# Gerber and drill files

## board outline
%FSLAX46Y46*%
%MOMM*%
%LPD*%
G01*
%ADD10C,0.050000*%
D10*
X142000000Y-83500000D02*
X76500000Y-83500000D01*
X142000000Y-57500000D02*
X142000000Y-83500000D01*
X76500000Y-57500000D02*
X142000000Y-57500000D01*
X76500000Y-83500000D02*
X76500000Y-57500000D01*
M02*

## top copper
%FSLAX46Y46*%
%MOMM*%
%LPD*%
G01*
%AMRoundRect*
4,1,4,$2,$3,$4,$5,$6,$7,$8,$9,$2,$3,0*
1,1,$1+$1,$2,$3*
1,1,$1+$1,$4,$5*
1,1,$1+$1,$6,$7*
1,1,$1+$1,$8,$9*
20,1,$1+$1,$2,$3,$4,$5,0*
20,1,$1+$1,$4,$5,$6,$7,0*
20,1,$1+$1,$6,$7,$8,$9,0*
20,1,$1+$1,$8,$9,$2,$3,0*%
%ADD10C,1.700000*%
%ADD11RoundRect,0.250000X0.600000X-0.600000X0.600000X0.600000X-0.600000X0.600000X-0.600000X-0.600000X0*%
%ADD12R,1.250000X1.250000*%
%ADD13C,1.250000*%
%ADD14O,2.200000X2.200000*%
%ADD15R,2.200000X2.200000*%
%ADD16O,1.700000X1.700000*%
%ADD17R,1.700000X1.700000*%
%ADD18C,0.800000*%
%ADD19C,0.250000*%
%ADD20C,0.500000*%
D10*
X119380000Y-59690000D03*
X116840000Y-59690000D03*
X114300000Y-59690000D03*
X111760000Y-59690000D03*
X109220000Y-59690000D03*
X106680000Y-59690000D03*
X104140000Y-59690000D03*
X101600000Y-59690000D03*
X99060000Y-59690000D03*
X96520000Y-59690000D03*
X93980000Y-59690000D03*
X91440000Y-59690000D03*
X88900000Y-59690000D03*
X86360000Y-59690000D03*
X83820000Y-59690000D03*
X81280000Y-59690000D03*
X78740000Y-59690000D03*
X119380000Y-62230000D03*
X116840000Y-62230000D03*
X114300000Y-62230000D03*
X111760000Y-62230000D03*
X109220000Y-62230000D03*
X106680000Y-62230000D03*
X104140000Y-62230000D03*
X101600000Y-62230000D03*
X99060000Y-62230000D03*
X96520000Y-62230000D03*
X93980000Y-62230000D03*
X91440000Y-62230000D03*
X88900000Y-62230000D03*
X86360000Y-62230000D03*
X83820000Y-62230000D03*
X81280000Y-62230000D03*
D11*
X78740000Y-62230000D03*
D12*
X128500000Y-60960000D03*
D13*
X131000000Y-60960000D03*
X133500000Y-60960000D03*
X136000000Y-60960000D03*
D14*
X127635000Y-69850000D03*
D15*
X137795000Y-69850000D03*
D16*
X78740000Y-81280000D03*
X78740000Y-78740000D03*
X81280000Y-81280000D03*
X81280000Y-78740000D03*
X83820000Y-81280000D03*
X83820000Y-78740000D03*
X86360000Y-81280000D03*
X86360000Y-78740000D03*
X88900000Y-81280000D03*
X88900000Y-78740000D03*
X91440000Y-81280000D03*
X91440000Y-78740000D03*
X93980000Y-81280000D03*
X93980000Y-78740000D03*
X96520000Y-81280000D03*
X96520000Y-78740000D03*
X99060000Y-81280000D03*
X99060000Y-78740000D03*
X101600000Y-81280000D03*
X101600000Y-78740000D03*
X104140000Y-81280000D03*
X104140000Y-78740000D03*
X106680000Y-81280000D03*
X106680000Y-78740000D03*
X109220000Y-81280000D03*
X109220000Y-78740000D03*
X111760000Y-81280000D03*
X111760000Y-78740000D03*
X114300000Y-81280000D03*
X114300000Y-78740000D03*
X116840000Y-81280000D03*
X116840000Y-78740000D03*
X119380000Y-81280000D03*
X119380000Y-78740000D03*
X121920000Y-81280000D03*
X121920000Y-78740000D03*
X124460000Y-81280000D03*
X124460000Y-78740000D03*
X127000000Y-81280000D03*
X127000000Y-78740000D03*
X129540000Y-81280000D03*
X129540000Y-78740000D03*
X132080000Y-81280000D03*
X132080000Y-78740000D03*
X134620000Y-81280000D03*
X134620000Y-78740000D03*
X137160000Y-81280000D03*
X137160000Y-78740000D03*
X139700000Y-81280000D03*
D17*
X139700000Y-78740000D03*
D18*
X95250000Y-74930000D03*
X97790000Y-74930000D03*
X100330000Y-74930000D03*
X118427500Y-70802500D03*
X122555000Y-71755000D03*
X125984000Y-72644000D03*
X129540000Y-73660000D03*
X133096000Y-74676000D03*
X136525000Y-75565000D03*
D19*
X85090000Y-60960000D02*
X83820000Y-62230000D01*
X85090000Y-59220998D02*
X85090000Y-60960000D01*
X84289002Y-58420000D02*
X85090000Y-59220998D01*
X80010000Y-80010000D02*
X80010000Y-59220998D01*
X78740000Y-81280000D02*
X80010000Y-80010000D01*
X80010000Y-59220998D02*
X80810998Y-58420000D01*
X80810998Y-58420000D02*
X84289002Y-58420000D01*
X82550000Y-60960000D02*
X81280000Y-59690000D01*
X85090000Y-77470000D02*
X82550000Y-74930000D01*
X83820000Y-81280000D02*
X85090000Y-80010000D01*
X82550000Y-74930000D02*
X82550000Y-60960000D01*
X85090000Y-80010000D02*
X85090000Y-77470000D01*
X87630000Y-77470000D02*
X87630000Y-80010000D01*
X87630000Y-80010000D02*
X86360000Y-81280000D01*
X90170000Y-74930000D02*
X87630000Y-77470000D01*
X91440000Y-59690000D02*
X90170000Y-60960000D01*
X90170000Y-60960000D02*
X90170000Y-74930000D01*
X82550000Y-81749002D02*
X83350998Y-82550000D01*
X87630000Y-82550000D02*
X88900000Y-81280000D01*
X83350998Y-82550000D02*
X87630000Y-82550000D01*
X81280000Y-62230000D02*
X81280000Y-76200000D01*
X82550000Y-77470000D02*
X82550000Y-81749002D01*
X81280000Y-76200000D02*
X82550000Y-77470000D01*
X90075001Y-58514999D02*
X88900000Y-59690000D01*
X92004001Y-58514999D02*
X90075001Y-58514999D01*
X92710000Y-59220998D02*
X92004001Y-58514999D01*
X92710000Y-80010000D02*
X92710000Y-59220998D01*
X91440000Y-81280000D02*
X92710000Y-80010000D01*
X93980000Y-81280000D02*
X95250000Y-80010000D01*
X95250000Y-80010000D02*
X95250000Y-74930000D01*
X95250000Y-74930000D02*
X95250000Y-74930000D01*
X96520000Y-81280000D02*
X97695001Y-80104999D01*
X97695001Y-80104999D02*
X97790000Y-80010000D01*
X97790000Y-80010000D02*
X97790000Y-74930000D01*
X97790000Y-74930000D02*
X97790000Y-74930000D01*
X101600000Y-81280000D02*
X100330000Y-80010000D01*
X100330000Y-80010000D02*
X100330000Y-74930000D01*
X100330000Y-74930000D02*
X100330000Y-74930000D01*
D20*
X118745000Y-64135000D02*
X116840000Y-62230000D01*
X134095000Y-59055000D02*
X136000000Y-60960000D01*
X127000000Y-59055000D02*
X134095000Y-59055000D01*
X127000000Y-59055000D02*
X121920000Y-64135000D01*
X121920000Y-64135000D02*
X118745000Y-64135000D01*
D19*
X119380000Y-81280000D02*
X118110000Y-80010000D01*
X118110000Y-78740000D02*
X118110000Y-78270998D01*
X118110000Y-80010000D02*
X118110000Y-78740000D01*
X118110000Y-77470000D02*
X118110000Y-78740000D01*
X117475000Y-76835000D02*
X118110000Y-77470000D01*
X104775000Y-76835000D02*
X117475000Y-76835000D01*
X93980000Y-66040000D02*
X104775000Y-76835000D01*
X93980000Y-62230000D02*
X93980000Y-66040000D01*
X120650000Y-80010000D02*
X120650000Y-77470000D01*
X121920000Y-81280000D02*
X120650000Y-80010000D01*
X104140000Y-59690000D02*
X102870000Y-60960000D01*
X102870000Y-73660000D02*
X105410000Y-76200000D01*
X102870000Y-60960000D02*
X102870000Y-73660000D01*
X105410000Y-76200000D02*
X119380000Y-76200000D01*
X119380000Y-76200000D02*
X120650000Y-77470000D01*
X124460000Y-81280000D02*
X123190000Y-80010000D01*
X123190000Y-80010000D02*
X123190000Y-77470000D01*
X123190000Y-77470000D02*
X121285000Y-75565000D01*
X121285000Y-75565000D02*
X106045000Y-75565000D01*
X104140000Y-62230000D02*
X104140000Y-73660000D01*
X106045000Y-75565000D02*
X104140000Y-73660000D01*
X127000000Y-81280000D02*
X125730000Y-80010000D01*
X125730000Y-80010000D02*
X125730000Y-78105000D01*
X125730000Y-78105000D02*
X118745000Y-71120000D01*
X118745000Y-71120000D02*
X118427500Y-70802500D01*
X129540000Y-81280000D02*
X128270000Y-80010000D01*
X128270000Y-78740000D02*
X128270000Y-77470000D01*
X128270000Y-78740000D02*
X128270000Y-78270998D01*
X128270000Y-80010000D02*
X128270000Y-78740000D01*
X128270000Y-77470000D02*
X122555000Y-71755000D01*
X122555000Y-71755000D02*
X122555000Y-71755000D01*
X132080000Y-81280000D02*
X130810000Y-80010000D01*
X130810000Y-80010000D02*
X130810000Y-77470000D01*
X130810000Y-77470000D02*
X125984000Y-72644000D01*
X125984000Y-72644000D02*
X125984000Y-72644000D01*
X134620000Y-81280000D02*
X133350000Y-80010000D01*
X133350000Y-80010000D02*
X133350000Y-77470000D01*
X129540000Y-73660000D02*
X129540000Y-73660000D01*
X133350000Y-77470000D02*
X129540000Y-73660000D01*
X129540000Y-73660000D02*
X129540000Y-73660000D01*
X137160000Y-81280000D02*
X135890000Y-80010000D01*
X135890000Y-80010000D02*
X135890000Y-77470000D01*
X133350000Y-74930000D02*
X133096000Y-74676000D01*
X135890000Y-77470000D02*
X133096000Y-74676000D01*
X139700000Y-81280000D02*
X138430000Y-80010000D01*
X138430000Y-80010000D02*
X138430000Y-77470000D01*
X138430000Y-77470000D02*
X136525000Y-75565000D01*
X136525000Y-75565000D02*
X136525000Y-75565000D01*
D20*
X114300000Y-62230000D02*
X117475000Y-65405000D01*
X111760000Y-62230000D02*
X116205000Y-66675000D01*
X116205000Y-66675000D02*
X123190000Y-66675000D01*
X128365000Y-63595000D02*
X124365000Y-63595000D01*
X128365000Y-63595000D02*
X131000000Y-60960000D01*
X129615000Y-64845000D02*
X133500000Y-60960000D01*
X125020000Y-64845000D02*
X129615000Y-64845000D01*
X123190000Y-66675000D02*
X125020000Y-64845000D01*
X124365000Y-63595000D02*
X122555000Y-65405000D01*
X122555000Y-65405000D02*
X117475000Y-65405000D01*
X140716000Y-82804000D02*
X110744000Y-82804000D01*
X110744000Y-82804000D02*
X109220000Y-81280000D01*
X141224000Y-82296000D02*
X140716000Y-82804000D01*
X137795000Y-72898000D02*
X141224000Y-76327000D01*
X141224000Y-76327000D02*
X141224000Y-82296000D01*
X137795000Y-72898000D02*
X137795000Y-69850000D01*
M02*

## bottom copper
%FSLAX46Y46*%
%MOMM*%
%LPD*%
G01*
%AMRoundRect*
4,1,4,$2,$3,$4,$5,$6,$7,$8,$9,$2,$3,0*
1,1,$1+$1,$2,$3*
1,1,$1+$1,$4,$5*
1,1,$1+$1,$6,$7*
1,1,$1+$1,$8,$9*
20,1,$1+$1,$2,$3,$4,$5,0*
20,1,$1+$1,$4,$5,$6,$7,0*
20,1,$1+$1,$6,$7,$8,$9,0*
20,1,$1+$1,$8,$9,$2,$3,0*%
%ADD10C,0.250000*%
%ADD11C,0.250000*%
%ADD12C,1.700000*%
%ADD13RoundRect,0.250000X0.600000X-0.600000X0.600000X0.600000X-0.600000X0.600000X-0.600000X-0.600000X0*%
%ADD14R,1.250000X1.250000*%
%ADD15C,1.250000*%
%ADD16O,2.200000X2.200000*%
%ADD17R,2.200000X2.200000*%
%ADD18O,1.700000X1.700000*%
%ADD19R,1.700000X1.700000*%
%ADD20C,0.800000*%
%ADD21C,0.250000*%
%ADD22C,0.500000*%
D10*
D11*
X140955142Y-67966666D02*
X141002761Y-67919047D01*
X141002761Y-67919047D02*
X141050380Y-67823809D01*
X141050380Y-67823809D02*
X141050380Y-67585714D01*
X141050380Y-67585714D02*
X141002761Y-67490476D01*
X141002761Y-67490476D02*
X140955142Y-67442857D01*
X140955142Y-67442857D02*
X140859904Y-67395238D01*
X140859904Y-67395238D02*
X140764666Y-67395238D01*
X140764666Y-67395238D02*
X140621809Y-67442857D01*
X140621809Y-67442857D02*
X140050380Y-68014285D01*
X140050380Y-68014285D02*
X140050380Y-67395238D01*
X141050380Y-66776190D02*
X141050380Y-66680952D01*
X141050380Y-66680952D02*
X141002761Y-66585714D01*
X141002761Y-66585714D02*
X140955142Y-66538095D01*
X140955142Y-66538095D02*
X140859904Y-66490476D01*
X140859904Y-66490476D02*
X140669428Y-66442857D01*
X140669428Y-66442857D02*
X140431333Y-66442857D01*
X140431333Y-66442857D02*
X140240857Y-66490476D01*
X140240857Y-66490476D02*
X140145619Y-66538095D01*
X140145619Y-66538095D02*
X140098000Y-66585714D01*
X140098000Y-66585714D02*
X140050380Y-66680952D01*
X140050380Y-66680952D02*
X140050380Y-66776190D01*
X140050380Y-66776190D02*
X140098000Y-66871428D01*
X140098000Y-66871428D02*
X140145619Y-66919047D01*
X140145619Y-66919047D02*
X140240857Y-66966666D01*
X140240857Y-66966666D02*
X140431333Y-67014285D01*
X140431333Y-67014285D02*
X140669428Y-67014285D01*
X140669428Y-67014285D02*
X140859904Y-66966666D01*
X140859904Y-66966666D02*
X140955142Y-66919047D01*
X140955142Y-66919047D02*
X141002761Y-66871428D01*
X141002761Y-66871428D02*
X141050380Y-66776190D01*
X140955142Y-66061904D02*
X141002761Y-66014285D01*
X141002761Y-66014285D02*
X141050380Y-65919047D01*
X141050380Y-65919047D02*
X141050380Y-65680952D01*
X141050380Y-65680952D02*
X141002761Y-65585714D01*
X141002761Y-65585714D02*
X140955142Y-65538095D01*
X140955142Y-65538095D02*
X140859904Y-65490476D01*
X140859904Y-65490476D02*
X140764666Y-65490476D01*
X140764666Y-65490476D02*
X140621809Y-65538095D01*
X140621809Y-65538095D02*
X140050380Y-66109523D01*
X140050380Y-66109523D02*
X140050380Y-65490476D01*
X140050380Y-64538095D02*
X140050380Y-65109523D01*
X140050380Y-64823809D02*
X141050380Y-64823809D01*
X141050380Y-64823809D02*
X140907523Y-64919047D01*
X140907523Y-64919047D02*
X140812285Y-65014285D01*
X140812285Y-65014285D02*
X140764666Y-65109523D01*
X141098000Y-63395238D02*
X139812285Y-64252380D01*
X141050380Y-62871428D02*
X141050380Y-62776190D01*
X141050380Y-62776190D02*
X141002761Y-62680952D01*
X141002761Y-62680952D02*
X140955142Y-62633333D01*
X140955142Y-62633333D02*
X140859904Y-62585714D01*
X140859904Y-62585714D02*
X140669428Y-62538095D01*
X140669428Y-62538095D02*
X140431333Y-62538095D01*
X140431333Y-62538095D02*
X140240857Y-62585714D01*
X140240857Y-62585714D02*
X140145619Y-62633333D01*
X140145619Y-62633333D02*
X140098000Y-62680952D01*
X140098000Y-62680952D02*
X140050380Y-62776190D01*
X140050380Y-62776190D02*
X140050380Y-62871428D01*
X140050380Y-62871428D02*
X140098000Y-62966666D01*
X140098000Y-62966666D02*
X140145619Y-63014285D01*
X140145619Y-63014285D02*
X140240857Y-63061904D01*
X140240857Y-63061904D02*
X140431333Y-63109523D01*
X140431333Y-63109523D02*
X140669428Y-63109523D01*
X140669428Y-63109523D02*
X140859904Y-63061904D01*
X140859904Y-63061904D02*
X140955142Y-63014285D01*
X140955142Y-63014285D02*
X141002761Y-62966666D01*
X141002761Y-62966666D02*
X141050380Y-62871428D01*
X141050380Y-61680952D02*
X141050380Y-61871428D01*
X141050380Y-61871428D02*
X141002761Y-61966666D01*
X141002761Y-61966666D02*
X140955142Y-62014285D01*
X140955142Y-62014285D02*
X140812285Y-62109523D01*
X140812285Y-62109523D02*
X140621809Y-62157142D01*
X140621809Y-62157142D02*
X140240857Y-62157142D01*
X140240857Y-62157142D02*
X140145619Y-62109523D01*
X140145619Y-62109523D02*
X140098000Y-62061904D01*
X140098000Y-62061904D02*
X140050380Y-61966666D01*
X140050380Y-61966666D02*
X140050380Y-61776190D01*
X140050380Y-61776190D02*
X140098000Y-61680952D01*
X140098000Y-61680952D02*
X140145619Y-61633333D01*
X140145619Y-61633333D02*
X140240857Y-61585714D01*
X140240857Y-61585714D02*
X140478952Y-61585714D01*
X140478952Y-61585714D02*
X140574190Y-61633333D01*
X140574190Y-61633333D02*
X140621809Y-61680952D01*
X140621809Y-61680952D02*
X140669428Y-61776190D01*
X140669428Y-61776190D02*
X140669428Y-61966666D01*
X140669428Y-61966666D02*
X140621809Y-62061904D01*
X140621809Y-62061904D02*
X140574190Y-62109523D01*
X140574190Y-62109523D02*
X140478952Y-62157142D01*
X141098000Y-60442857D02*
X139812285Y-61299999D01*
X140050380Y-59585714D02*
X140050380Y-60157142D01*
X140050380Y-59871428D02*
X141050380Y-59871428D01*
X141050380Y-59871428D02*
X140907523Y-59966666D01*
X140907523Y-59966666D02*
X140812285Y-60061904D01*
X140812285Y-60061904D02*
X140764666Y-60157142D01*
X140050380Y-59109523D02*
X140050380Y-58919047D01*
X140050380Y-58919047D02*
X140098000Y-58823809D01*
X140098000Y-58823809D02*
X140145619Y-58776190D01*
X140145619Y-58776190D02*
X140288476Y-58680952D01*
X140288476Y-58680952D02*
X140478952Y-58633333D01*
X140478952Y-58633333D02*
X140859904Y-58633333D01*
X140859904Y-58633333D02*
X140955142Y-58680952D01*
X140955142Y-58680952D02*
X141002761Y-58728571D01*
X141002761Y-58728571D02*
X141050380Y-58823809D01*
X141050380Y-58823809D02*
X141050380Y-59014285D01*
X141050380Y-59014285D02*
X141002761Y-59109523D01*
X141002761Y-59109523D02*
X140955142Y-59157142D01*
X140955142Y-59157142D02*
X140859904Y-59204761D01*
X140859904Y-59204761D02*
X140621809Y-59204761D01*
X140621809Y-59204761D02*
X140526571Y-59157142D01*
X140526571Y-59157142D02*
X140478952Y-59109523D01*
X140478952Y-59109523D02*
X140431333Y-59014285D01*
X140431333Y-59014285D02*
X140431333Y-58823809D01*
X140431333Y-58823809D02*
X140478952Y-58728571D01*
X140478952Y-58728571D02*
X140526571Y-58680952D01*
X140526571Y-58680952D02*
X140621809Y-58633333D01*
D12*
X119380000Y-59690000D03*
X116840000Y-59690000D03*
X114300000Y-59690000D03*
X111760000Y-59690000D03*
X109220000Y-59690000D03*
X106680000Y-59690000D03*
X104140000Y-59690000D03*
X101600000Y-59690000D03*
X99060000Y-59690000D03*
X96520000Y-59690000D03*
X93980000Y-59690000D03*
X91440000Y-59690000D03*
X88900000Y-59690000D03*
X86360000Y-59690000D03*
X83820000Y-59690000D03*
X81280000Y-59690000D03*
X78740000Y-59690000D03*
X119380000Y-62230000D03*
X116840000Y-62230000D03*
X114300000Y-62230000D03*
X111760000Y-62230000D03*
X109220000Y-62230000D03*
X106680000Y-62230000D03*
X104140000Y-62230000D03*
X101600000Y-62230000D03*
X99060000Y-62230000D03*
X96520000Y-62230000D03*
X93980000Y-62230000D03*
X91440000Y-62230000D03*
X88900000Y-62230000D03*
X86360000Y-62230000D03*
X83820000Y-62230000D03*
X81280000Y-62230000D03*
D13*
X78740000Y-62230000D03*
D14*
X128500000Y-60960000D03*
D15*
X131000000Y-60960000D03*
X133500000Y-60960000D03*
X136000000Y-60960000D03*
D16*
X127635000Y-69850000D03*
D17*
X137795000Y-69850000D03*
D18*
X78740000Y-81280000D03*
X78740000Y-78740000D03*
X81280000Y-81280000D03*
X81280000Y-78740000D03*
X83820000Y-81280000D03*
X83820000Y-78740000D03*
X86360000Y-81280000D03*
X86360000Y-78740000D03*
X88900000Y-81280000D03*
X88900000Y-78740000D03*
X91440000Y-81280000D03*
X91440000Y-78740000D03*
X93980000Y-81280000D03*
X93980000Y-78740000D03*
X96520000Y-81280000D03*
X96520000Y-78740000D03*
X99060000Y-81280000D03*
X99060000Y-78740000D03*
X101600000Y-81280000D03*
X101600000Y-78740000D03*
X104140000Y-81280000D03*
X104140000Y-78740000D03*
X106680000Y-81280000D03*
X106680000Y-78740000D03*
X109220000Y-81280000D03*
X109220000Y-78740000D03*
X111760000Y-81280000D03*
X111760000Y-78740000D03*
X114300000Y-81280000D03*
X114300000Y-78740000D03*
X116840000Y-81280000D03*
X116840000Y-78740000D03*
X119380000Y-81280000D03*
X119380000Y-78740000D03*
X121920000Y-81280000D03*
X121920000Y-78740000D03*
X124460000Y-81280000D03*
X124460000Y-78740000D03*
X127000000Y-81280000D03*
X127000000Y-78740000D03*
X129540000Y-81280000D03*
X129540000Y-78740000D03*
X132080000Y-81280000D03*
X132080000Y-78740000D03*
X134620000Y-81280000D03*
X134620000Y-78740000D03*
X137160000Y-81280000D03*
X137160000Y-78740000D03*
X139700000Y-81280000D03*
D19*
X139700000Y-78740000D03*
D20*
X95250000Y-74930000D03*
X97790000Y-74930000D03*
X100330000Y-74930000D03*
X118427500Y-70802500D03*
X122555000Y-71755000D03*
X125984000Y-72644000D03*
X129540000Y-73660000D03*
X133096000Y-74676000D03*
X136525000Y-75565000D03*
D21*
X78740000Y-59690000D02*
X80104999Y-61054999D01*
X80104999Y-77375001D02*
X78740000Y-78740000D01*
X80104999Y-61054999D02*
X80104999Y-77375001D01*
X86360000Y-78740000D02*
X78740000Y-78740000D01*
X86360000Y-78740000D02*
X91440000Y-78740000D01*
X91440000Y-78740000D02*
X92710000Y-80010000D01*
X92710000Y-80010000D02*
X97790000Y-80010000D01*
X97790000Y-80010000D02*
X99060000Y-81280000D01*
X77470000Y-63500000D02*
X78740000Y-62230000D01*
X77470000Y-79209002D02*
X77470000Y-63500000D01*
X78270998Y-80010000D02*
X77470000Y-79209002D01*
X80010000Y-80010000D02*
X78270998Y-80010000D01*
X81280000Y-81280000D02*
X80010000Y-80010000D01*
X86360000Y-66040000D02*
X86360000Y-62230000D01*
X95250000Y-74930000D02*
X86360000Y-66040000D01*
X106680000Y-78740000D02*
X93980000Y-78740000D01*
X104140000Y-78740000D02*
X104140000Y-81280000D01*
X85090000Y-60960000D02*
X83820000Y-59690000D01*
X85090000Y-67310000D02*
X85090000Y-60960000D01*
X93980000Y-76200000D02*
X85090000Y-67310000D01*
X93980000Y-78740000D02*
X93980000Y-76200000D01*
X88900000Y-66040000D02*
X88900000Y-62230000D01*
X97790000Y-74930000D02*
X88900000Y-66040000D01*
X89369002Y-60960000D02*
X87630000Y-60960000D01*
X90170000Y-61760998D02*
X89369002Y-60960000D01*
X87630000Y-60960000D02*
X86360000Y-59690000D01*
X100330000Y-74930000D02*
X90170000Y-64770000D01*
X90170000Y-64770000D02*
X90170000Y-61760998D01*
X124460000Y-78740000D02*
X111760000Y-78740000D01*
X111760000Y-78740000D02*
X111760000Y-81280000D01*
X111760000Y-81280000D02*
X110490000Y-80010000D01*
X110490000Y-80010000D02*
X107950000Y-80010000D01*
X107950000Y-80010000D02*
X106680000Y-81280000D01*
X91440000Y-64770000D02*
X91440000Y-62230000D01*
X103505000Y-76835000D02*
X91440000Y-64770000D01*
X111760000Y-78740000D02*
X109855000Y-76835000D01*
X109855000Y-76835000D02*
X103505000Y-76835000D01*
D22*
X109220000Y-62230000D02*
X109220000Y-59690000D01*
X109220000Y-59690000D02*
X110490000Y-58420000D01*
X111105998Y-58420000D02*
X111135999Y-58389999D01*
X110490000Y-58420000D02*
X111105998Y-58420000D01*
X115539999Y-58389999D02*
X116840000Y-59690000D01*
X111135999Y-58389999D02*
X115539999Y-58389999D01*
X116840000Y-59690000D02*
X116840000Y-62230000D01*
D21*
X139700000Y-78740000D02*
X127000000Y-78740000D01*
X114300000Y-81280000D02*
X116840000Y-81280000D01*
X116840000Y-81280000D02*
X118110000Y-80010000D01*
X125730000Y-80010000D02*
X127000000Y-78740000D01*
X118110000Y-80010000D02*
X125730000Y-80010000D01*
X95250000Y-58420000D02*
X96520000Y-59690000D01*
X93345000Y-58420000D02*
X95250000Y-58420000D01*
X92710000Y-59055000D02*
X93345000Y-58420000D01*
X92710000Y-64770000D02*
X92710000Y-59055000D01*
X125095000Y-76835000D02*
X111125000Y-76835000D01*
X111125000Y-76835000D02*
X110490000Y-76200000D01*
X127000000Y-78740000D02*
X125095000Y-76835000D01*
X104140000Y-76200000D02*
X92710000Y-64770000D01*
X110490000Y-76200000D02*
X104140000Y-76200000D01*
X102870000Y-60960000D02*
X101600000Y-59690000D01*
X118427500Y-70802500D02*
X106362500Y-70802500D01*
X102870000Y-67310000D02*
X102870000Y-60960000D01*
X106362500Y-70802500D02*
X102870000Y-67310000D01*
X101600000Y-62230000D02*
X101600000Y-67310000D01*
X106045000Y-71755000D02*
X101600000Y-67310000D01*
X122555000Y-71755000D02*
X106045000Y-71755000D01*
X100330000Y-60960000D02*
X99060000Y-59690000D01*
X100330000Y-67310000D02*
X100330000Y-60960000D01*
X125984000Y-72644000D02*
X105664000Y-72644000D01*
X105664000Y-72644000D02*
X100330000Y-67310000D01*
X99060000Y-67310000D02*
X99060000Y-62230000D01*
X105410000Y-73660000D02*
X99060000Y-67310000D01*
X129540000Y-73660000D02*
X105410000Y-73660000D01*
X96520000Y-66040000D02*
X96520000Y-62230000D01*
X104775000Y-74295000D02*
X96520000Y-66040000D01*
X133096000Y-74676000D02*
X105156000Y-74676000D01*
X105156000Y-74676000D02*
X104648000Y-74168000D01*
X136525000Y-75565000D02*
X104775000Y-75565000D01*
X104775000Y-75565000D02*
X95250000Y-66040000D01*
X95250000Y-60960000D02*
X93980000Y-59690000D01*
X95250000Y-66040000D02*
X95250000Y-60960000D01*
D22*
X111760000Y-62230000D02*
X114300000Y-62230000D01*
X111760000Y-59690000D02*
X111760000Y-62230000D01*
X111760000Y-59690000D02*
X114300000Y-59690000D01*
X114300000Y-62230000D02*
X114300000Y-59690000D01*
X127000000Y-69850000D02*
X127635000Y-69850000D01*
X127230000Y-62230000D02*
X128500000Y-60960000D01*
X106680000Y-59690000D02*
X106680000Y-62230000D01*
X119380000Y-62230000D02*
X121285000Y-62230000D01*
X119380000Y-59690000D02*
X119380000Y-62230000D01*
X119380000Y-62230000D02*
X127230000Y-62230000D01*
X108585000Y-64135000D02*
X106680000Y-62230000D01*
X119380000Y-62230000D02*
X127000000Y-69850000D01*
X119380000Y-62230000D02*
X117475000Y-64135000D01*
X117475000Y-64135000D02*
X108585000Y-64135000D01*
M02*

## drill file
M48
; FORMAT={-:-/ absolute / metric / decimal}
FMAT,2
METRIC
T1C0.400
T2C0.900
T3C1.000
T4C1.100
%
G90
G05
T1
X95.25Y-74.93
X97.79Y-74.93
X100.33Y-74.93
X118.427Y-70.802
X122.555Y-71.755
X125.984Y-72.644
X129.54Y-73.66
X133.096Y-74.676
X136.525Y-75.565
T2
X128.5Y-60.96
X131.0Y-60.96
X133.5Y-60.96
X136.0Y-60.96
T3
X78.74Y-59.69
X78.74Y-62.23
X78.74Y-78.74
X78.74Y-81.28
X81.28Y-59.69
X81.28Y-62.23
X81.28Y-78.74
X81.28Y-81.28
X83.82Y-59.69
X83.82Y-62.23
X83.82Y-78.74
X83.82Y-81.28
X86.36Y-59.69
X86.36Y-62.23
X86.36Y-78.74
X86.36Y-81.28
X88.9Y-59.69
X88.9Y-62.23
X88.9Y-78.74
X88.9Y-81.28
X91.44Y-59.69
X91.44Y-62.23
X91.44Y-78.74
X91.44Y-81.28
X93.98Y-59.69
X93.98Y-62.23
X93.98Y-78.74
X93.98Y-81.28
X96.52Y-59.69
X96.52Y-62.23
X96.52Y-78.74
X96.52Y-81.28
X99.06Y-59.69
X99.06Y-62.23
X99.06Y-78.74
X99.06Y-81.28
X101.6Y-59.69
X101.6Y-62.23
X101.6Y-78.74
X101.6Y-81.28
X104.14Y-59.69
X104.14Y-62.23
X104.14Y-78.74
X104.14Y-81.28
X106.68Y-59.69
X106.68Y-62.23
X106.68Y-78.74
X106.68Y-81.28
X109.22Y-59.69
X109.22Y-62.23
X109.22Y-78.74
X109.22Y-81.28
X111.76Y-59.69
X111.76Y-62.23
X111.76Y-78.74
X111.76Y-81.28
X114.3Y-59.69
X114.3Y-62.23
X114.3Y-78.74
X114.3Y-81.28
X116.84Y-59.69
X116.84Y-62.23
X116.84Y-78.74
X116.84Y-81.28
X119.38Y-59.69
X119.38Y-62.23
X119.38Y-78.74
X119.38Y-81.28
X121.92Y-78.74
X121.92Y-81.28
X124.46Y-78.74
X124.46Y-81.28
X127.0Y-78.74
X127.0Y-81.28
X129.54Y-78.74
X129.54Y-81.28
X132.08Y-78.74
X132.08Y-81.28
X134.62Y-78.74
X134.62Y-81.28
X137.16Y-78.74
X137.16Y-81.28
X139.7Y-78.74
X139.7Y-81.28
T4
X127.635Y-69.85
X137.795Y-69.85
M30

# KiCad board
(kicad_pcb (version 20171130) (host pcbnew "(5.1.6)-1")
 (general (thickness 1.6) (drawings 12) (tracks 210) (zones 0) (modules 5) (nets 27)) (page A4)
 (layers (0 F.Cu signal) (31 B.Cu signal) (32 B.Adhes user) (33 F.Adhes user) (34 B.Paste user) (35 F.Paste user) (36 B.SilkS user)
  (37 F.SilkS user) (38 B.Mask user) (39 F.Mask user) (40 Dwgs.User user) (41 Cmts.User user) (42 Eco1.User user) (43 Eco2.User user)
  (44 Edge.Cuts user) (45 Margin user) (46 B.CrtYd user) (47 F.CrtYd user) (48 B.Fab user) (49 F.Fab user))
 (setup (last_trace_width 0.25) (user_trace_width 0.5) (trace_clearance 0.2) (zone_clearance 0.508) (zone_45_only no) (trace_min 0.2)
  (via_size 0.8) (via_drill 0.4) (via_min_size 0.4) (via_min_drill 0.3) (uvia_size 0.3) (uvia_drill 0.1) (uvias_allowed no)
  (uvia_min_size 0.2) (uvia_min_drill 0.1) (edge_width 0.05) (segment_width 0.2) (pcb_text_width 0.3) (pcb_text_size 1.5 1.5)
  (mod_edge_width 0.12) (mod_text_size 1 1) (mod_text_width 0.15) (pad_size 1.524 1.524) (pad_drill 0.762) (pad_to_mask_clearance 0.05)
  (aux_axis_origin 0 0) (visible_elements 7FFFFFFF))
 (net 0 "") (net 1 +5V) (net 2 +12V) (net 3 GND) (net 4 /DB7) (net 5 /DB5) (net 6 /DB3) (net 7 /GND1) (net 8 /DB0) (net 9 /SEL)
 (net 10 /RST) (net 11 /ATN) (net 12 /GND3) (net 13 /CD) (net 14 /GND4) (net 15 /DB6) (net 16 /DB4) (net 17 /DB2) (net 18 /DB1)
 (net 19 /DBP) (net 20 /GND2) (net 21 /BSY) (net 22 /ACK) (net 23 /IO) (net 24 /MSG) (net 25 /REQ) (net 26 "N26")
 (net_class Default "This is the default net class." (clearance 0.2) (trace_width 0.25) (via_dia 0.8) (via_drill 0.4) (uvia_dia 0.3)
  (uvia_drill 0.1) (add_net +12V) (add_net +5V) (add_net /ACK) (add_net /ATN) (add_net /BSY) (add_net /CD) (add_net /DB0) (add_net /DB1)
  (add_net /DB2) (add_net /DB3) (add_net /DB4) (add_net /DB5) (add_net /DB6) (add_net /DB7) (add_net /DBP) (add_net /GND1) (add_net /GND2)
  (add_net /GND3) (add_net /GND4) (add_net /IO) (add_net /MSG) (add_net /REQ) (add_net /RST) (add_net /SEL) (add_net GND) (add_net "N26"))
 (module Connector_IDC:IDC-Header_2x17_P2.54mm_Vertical (layer F.Cu) (at 78.74 62.23 90)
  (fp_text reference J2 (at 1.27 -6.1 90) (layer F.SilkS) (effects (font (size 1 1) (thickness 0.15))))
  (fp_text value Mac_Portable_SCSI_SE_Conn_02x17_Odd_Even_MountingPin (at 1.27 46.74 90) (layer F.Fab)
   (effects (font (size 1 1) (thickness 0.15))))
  (pad 34 thru_hole circle (at 2.54 40.64 90) (size 1.7 1.7) (drill 1) (layers *.Cu *.Mask) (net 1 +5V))
  (pad 32 thru_hole circle (at 2.54 38.1 90) (size 1.7 1.7) (drill 1) (layers *.Cu *.Mask) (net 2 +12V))
  (pad 30 thru_hole circle (at 2.54 35.56 90) (size 1.7 1.7) (drill 1) (layers *.Cu *.Mask) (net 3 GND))
  (pad 28 thru_hole circle (at 2.54 33.02 90) (size 1.7 1.7) (drill 1) (layers *.Cu *.Mask) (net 3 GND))
  (pad 26 thru_hole circle (at 2.54 30.48 90) (size 1.7 1.7) (drill 1) (layers *.Cu *.Mask) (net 2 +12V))
  (pad 24 thru_hole circle (at 2.54 27.94 90) (size 1.7 1.7) (drill 1) (layers *.Cu *.Mask) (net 1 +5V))
  (pad 22 thru_hole circle (at 2.54 25.4 90) (size 1.7 1.7) (drill 1) (layers *.Cu *.Mask) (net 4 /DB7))
  (pad 20 thru_hole circle (at 2.54 22.86 90) (size 1.7 1.7) (drill 1) (layers *.Cu *.Mask) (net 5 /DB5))
  (pad 18 thru_hole circle (at 2.54 20.32 90) (size 1.7 1.7) (drill 1) (layers *.Cu *.Mask) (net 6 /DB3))
  (pad 16 thru_hole circle (at 2.54 17.78 90) (size 1.7 1.7) (drill 1) (layers *.Cu *.Mask) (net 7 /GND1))
  (pad 14 thru_hole circle (at 2.54 15.24 90) (size 1.7 1.7) (drill 1) (layers *.Cu *.Mask) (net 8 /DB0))
  (pad 12 thru_hole circle (at 2.54 12.7 90) (size 1.7 1.7) (drill 1) (layers *.Cu *.Mask) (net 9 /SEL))
  (pad 10 thru_hole circle (at 2.54 10.16 90) (size 1.7 1.7) (drill 1) (layers *.Cu *.Mask) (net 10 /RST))
  (pad 8 thru_hole circle (at 2.54 7.62 90) (size 1.7 1.7) (drill 1) (layers *.Cu *.Mask) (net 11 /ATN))
  (pad 6 thru_hole circle (at 2.54 5.08 90) (size 1.7 1.7) (drill 1) (layers *.Cu *.Mask) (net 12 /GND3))
  (pad 4 thru_hole circle (at 2.54 2.54 90) (size 1.7 1.7) (drill 1) (layers *.Cu *.Mask) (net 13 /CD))
  (pad 2 thru_hole circle (at 2.54 0 90) (size 1.7 1.7) (drill 1) (layers *.Cu *.Mask) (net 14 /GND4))
  (pad 33 thru_hole circle (at 0 40.64 90) (size 1.7 1.7) (drill 1) (layers *.Cu *.Mask) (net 1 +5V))
  (pad 31 thru_hole circle (at 0 38.1 90) (size 1.7 1.7) (drill 1) (layers *.Cu *.Mask) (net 2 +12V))
  (pad 29 thru_hole circle (at 0 35.56 90) (size 1.7 1.7) (drill 1) (layers *.Cu *.Mask) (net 3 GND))
  (pad 27 thru_hole circle (at 0 33.02 90) (size 1.7 1.7) (drill 1) (layers *.Cu *.Mask) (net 3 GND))
  (pad 25 thru_hole circle (at 0 30.48 90) (size 1.7 1.7) (drill 1) (layers *.Cu *.Mask) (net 2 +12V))
  (pad 23 thru_hole circle (at 0 27.94 90) (size 1.7 1.7) (drill 1) (layers *.Cu *.Mask) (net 1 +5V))
  (pad 21 thru_hole circle (at 0 25.4 90) (size 1.7 1.7) (drill 1) (layers *.Cu *.Mask) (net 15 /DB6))
  (pad 19 thru_hole circle (at 0 22.86 90) (size 1.7 1.7) (drill 1) (layers *.Cu *.Mask) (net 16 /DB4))
  (pad 17 thru_hole circle (at 0 20.32 90) (size 1.7 1.7) (drill 1) (layers *.Cu *.Mask) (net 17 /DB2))
  (pad 15 thru_hole circle (at 0 17.78 90) (size 1.7 1.7) (drill 1) (layers *.Cu *.Mask) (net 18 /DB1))
  (pad 13 thru_hole circle (at 0 15.24 90) (size 1.7 1.7) (drill 1) (layers *.Cu *.Mask) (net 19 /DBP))
  (pad 11 thru_hole circle (at 0 12.7 90) (size 1.7 1.7) (drill 1) (layers *.Cu *.Mask) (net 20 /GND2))
  (pad 9 thru_hole circle (at 0 10.16 90) (size 1.7 1.7) (drill 1) (layers *.Cu *.Mask) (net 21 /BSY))
  (pad 7 thru_hole circle (at 0 7.62 90) (size 1.7 1.7) (drill 1) (layers *.Cu *.Mask) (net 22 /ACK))
  (pad 5 thru_hole circle (at 0 5.08 90) (size 1.7 1.7) (drill 1) (layers *.Cu *.Mask) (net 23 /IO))
  (pad 3 thru_hole circle (at 0 2.54 90) (size 1.7 1.7) (drill 1) (layers *.Cu *.Mask) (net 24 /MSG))
  (pad 1 thru_hole roundrect (at 0 0 90) (size 1.7 1.7) (drill 1) (layers *.Cu *.Mask) (roundrect_rratio 0.147059) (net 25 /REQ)))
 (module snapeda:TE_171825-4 (layer F.Cu) (at 128.5 60.96)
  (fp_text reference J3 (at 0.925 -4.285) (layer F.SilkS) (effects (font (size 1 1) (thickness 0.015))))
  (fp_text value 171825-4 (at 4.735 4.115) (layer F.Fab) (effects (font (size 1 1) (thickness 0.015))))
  (pad 1 thru_hole rect (at 0 0) (size 1.25 1.25) (drill 0.9) (layers *.Cu *.Mask) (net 1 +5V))
  (pad 2 thru_hole circle (at 2.5 0) (size 1.25 1.25) (drill 0.9) (layers *.Cu *.Mask) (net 3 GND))
  (pad 3 thru_hole circle (at 5 0) (size 1.25 1.25) (drill 0.9) (layers *.Cu *.Mask) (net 3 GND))
  (pad 4 thru_hole circle (at 7.5 0) (size 1.25 1.25) (drill 0.9) (layers *.Cu *.Mask) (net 2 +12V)))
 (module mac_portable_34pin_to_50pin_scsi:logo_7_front (layer F.Cu) (at 89.7 70.9)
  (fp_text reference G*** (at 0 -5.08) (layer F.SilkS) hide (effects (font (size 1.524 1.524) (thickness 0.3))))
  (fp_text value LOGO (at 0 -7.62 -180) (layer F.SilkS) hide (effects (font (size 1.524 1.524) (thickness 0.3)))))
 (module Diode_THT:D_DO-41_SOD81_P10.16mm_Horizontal (layer F.Cu) (at 137.795 69.85 180)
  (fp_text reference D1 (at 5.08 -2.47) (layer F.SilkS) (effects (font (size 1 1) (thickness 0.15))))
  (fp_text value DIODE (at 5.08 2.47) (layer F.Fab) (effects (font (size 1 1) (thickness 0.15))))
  (pad 2 thru_hole oval (at 10.16 0 180) (size 2.2 2.2) (drill 1.1) (layers *.Cu *.Mask) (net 1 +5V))
  (pad 1 thru_hole rect (at 0 0 180) (size 2.2 2.2) (drill 1.1) (layers *.Cu *.Mask) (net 1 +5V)))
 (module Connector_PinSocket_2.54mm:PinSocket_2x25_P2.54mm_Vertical (layer B.Cu) (at 139.7 78.74 90)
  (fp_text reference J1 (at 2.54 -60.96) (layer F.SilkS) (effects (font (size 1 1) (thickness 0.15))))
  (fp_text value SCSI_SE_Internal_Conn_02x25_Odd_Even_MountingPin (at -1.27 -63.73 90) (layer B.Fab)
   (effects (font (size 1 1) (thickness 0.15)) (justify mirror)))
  (pad 50 thru_hole oval (at -2.54 -60.96 90) (size 1.7 1.7) (drill 1) (layers *.Cu *.Mask) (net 23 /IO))
  (pad 49 thru_hole oval (at 0 -60.96 90) (size 1.7 1.7) (drill 1) (layers *.Cu *.Mask) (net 14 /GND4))
  (pad 48 thru_hole oval (at -2.54 -58.42 90) (size 1.7 1.7) (drill 1) (layers *.Cu *.Mask) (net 25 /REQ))
  (pad 47 thru_hole oval (at 0 -58.42 90) (size 1.7 1.7) (drill 1) (layers *.Cu *.Mask) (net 14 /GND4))
  (pad 46 thru_hole oval (at -2.54 -55.88 90) (size 1.7 1.7) (drill 1) (layers *.Cu *.Mask) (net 13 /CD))
  (pad 45 thru_hole oval (at 0 -55.88 90) (size 1.7 1.7) (drill 1) (layers *.Cu *.Mask) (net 14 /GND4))
  (pad 44 thru_hole oval (at -2.54 -53.34 90) (size 1.7 1.7) (drill 1) (layers *.Cu *.Mask) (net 9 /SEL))
  (pad 43 thru_hole oval (at 0 -53.34 90) (size 1.7 1.7) (drill 1) (layers *.Cu *.Mask) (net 14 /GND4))
  (pad 42 thru_hole oval (at -2.54 -50.8 90) (size 1.7 1.7) (drill 1) (layers *.Cu *.Mask) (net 24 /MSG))
  (pad 41 thru_hole oval (at 0 -50.8 90) (size 1.7 1.7) (drill 1) (layers *.Cu *.Mask) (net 14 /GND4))
  (pad 40 thru_hole oval (at -2.54 -48.26 90) (size 1.7 1.7) (drill 1) (layers *.Cu *.Mask) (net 10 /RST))
  (pad 39 thru_hole oval (at 0 -48.26 90) (size 1.7 1.7) (drill 1) (layers *.Cu *.Mask) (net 14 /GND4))
  (pad 38 thru_hole oval (at -2.54 -45.72 90) (size 1.7 1.7) (drill 1) (layers *.Cu *.Mask) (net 22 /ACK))
  (pad 37 thru_hole oval (at 0 -45.72 90) (size 1.7 1.7) (drill 1) (layers *.Cu *.Mask) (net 12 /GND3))
  (pad 36 thru_hole oval (at -2.54 -43.18 90) (size 1.7 1.7) (drill 1) (layers *.Cu *.Mask) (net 21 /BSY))
  (pad 35 thru_hole oval (at 0 -43.18 90) (size 1.7 1.7) (drill 1) (layers *.Cu *.Mask) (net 12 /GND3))
  (pad 34 thru_hole oval (at -2.54 -40.64 90) (size 1.7 1.7) (drill 1) (layers *.Cu *.Mask) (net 14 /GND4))
  (pad 33 thru_hole oval (at 0 -40.64 90) (size 1.7 1.7) (drill 1) (layers *.Cu *.Mask) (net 12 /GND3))
  (pad 32 thru_hole oval (at -2.54 -38.1 90) (size 1.7 1.7) (drill 1) (layers *.Cu *.Mask) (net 11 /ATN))
  (pad 31 thru_hole oval (at 0 -38.1 90) (size 1.7 1.7) (drill 1) (layers *.Cu *.Mask) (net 12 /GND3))
  (pad 30 thru_hole oval (at -2.54 -35.56 90) (size 1.7 1.7) (drill 1) (layers *.Cu *.Mask) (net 12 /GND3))
  (pad 29 thru_hole oval (at 0 -35.56 90) (size 1.7 1.7) (drill 1) (layers *.Cu *.Mask) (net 12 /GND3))
  (pad 28 thru_hole oval (at -2.54 -33.02 90) (size 1.7 1.7) (drill 1) (layers *.Cu *.Mask) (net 20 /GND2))
  (pad 27 thru_hole oval (at 0 -33.02 90) (size 1.7 1.7) (drill 1) (layers *.Cu *.Mask) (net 12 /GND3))
  (pad 26 thru_hole oval (at -2.54 -30.48 90) (size 1.7 1.7) (drill 1) (layers *.Cu *.Mask) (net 1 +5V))
  (pad 25 thru_hole oval (at 0 -30.48 90) (size 1.7 1.7) (drill 1) (layers *.Cu *.Mask) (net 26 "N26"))
  (pad 24 thru_hole oval (at -2.54 -27.94 90) (size 1.7 1.7) (drill 1) (layers *.Cu *.Mask) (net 20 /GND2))
  (pad 23 thru_hole oval (at 0 -27.94 90) (size 1.7 1.7) (drill 1) (layers *.Cu *.Mask) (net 20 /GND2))
  (pad 22 thru_hole oval (at -2.54 -25.4 90) (size 1.7 1.7) (drill 1) (layers *.Cu *.Mask) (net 7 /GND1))
  (pad 21 thru_hole oval (at 0 -25.4 90) (size 1.7 1.7) (drill 1) (layers *.Cu *.Mask) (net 20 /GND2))
  (pad 20 thru_hole oval (at -2.54 -22.86 90) (size 1.7 1.7) (drill 1) (layers *.Cu *.Mask) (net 7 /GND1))
  (pad 19 thru_hole oval (at 0 -22.86 90) (size 1.7 1.7) (drill 1) (layers *.Cu *.Mask) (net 20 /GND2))
  (pad 18 thru_hole oval (at -2.54 -20.32 90) (size 1.7 1.7) (drill 1) (layers *.Cu *.Mask) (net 19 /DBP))
  (pad 17 thru_hole oval (at 0 -20.32 90) (size 1.7 1.7) (drill 1) (layers *.Cu *.Mask) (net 20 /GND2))
  (pad 16 thru_hole oval (at -2.54 -17.78 90) (size 1.7 1.7) (drill 1) (layers *.Cu *.Mask) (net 4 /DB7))
  (pad 15 thru_hole oval (at 0 -17.78 90) (size 1.7 1.7) (drill 1) (layers *.Cu *.Mask) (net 20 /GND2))
  (pad 14 thru_hole oval (at -2.54 -15.24 90) (size 1.7 1.7) (drill 1) (layers *.Cu *.Mask) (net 15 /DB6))
  (pad 13 thru_hole oval (at 0 -15.24 90) (size 1.7 1.7) (drill 1) (layers *.Cu *.Mask) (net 20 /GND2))
  (pad 12 thru_hole oval (at -2.54 -12.7 90) (size 1.7 1.7) (drill 1) (layers *.Cu *.Mask) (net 5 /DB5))
  (pad 11 thru_hole oval (at 0 -12.7 90) (size 1.7 1.7) (drill 1) (layers *.Cu *.Mask) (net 7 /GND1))
  (pad 10 thru_hole oval (at -2.54 -10.16 90) (size 1.7 1.7) (drill 1) (layers *.Cu *.Mask) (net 16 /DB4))
  (pad 9 thru_hole oval (at 0 -10.16 90) (size 1.7 1.7) (drill 1) (layers *.Cu *.Mask) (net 7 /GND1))
  (pad 8 thru_hole oval (at -2.54 -7.62 90) (size 1.7 1.7) (drill 1) (layers *.Cu *.Mask) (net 6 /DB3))
  (pad 7 thru_hole oval (at 0 -7.62 90) (size 1.7 1.7) (drill 1) (layers *.Cu *.Mask) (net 7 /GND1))
  (pad 6 thru_hole oval (at -2.54 -5.08 90) (size 1.7 1.7) (drill 1) (layers *.Cu *.Mask) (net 17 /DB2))
  (pad 5 thru_hole oval (at 0 -5.08 90) (size 1.7 1.7) (drill 1) (layers *.Cu *.Mask) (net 7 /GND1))
  (pad 4 thru_hole oval (at -2.54 -2.54 90) (size 1.7 1.7) (drill 1) (layers *.Cu *.Mask) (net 18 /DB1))
  (pad 3 thru_hole oval (at 0 -2.54 90) (size 1.7 1.7) (drill 1) (layers *.Cu *.Mask) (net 7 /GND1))
  (pad 2 thru_hole oval (at -2.54 0 90) (size 1.7 1.7) (drill 1) (layers *.Cu *.Mask) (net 8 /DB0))
  (pad 1 thru_hole rect (at 0 0 90) (size 1.7 1.7) (drill 1) (layers *.Cu *.Mask) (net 7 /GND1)))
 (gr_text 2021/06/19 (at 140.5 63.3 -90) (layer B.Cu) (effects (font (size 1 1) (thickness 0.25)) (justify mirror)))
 (gr_line (start 142 83.5) (end 76.5 83.5) (layer Edge.Cuts) (width 0.05))
 (gr_line (start 142 57.5) (end 142 83.5) (layer Edge.Cuts) (width 0.05))
 (gr_line (start 76.5 57.5) (end 142 57.5) (layer Edge.Cuts) (width 0.05))
 (gr_line (start 76.5 83.5) (end 76.5 57.5) (layer Edge.Cuts) (width 0.05))
 (segment (start 85.09 60.96) (end 83.82 62.23) (width 0.25) (layer F.Cu) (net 23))
 (segment (start 85.09 59.220998) (end 85.09 60.96) (width 0.25) (layer F.Cu) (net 23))
 (segment (start 84.289002 58.42) (end 85.09 59.220998) (width 0.25) (layer F.Cu) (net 23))
 (segment (start 80.01 80.01) (end 80.01 59.220998) (width 0.25) (layer F.Cu) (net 23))
 (segment (start 78.74 81.28) (end 80.01 80.01) (width 0.25) (layer F.Cu) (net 23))
 (segment (start 80.01 59.220998) (end 80.810998 58.42) (width 0.25) (layer F.Cu) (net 23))
 (segment (start 80.810998 58.42) (end 84.289002 58.42) (width 0.25) (layer F.Cu) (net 23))
 (segment (start 78.74 59.69) (end 80.104999 61.054999) (width 0.25) (layer B.Cu) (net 14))
 (segment (start 80.104999 77.375001) (end 78.74 78.74) (width 0.25) (layer B.Cu) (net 14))
 (segment (start 80.104999 61.054999) (end 80.104999 77.375001) (width 0.25) (layer B.Cu) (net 14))
 (segment (start 86.36 78.74) (end 78.74 78.74) (width 0.25) (layer B.Cu) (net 14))
 (segment (start 86.36 78.74) (end 91.44 78.74) (width 0.25) (layer B.Cu) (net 14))
 (segment (start 91.44 78.74) (end 92.71 80.01) (width 0.25) (layer B.Cu) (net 14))
 (segment (start 92.71 80.01) (end 97.79 80.01) (width 0.25) (layer B.Cu) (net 14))
 (segment (start 97.79 80.01) (end 99.06 81.28) (width 0.25) (layer B.Cu) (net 14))
 (segment (start 77.47 63.5) (end 78.74 62.23) (width 0.25) (layer B.Cu) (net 25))
 (segment (start 77.47 79.209002) (end 77.47 63.5) (width 0.25) (layer B.Cu) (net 25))
 (segment (start 78.270998 80.01) (end 77.47 79.209002) (width 0.25) (layer B.Cu) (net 25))
 (segment (start 80.01 80.01) (end 78.270998 80.01) (width 0.25) (layer B.Cu) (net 25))
 (segment (start 81.28 81.28) (end 80.01 80.01) (width 0.25) (layer B.Cu) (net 25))
 (segment (start 82.55 60.96) (end 81.28 59.69) (width 0.25) (layer F.Cu) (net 13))
 (segment (start 85.09 77.47) (end 82.55 74.93) (width 0.25) (layer F.Cu) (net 13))
 (segment (start 83.82 81.28) (end 85.09 80.01) (width 0.25) (layer F.Cu) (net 13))
 (segment (start 82.55 74.93) (end 82.55 60.96) (width 0.25) (layer F.Cu) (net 13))
 (segment (start 85.09 80.01) (end 85.09 77.47) (width 0.25) (layer F.Cu) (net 13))
 (segment (start 87.63 77.47) (end 87.63 80.01) (width 0.25) (layer F.Cu) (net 9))
 (segment (start 87.63 80.01) (end 86.36 81.28) (width 0.25) (layer F.Cu) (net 9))
 (segment (start 90.17 74.93) (end 87.63 77.47) (width 0.25) (layer F.Cu) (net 9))
 (segment (start 91.44 59.69) (end 90.17 60.96) (width 0.25) (layer F.Cu) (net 9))
 (segment (start 90.17 60.96) (end 90.17 74.93) (width 0.25) (layer F.Cu) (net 9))
 (segment (start 82.55 81.749002) (end 83.350998 82.55) (width 0.25) (layer F.Cu) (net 24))
 (segment (start 87.63 82.55) (end 88.9 81.28) (width 0.25) (layer F.Cu) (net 24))
 (segment (start 83.350998 82.55) (end 87.63 82.55) (width 0.25) (layer F.Cu) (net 24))
 (segment (start 81.28 62.23) (end 81.28 76.2) (width 0.25) (layer F.Cu) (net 24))
 (segment (start 82.55 77.47) (end 82.55 81.749002) (width 0.25) (layer F.Cu) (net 24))
 (segment (start 81.28 76.2) (end 82.55 77.47) (width 0.25) (layer F.Cu) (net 24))
 (segment (start 90.075001 58.514999) (end 88.9 59.69) (width 0.25) (layer F.Cu) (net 10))
 (segment (start 92.004001 58.514999) (end 90.075001 58.514999) (width 0.25) (layer F.Cu) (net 10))
 (segment (start 92.71 59.220998) (end 92.004001 58.514999) (width 0.25) (layer F.Cu) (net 10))
 (segment (start 92.71 80.01) (end 92.71 59.220998) (width 0.25) (layer F.Cu) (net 10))
 (segment (start 91.44 81.28) (end 92.71 80.01) (width 0.25) (layer F.Cu) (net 10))
 (segment (start 93.98 81.28) (end 95.25 80.01) (width 0.25) (layer F.Cu) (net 22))
 (segment (start 95.25 80.01) (end 95.25 74.93) (width 0.25) (layer F.Cu) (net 22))
 (segment (start 95.25 74.93) (end 95.25 74.93) (width 0.25) (layer F.Cu) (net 22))
 (via (at 95.25 74.93) (size 0.8) (drill 0.4) (layers F.Cu B.Cu) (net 22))
 (segment (start 86.36 66.04) (end 86.36 62.23) (width 0.25) (layer B.Cu) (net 22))
 (segment (start 95.25 74.93) (end 86.36 66.04) (width 0.25) (layer B.Cu) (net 22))
 (segment (start 106.68 78.74) (end 93.98 78.74) (width 0.25) (layer B.Cu) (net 12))
 (segment (start 104.14 78.74) (end 104.14 81.28) (width 0.25) (layer B.Cu) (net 12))
 (segment (start 85.09 60.96) (end 83.82 59.69) (width 0.25) (layer B.Cu) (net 12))
 (segment (start 85.09 67.31) (end 85.09 60.96) (width 0.25) (layer B.Cu) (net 12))
 (segment (start 93.98 76.2) (end 85.09 67.31) (width 0.25) (layer B.Cu) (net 12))
 (segment (start 93.98 78.74) (end 93.98 76.2) (width 0.25) (layer B.Cu) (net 12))
 (segment (start 96.52 81.28) (end 97.695001 80.104999) (width 0.25) (layer F.Cu) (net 21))
 (segment (start 97.695001 80.104999) (end 97.79 80.01) (width 0.25) (layer F.Cu) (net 21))
 (segment (start 97.79 80.01) (end 97.79 74.93) (width 0.25) (layer F.Cu) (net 21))
 (segment (start 97.79 74.93) (end 97.79 74.93) (width 0.25) (layer F.Cu) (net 21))
 (via (at 97.79 74.93) (size 0.8) (drill 0.4) (layers F.Cu B.Cu) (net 21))
 (segment (start 88.9 66.04) (end 88.9 62.23) (width 0.25) (layer B.Cu) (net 21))
 (segment (start 97.79 74.93) (end 88.9 66.04) (width 0.25) (layer B.Cu) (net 21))
 (segment (start 101.6 81.28) (end 100.33 80.01) (width 0.25) (layer F.Cu) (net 11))
 (segment (start 100.33 80.01) (end 100.33 74.93) (width 0.25) (layer F.Cu) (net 11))
 (segment (start 100.33 74.93) (end 100.33 74.93) (width 0.25) (layer F.Cu) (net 11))
 (via (at 100.33 74.93) (size 0.8) (drill 0.4) (layers F.Cu B.Cu) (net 11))
 (segment (start 89.369002 60.96) (end 87.63 60.96) (width 0.25) (layer B.Cu) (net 11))
 (segment (start 90.17 61.760998) (end 89.369002 60.96) (width 0.25) (layer B.Cu) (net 11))
 (segment (start 87.63 60.96) (end 86.36 59.69) (width 0.25) (layer B.Cu) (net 11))
 (segment (start 100.33 74.93) (end 90.17 64.77) (width 0.25) (layer B.Cu) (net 11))
 (segment (start 90.17 64.77) (end 90.17 61.760998) (width 0.25) (layer B.Cu) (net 11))
 (segment (start 124.46 78.74) (end 111.76 78.74) (width 0.25) (layer B.Cu) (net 20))
 (segment (start 111.76 78.74) (end 111.76 81.28) (width 0.25) (layer B.Cu) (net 20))
 (segment (start 111.76 81.28) (end 110.49 80.01) (width 0.25) (layer B.Cu) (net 20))
 (segment (start 110.49 80.01) (end 107.95 80.01) (width 0.25) (layer B.Cu) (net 20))
 (segment (start 107.95 80.01) (end 106.68 81.28) (width 0.25) (layer B.Cu) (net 20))
 (segment (start 91.44 64.77) (end 91.44 62.23) (width 0.25) (layer B.Cu) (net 20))
 (segment (start 103.505 76.835) (end 91.44 64.77) (width 0.25) (layer B.Cu) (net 20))
 (segment (start 111.76 78.74) (end 109.855 76.835) (width 0.25) (layer B.Cu) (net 20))
 (segment (start 109.855 76.835) (end 103.505 76.835) (width 0.25) (layer B.Cu) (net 20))
 (segment (start 109.22 62.23) (end 109.22 59.69) (width 0.5) (layer B.Cu) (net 2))
 (segment (start 109.22 59.69) (end 110.49 58.42) (width 0.5) (layer B.Cu) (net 2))
 (segment (start 111.105998 58.42) (end 111.135999 58.389999) (width 0.5) (layer B.Cu) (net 2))
 (segment (start 110.49 58.42) (end 111.105998 58.42) (width 0.5) (layer B.Cu) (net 2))
 (segment (start 115.539999 58.389999) (end 116.84 59.69) (width 0.5) (layer B.Cu) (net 2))
 (segment (start 111.135999 58.389999) (end 115.539999 58.389999) (width 0.5) (layer B.Cu) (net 2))
 (segment (start 116.84 59.69) (end 116.84 62.23) (width 0.5) (layer B.Cu) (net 2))
 (segment (start 118.745 64.135) (end 116.84 62.23) (width 0.5) (layer F.Cu) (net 2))
 (segment (start 134.095 59.055) (end 136 60.96) (width 0.5) (layer F.Cu) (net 2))
 (segment (start 127 59.055) (end 134.095 59.055) (width 0.5) (layer F.Cu) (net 2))
 (segment (start 127 59.055) (end 121.92 64.135) (width 0.5) (layer F.Cu) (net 2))
 (segment (start 121.92 64.135) (end 118.745 64.135) (width 0.5) (layer F.Cu) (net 2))
 (segment (start 139.7 78.74) (end 127 78.74) (width 0.25) (layer B.Cu) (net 7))
 (segment (start 114.3 81.28) (end 116.84 81.28) (width 0.25) (layer B.Cu) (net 7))
 (segment (start 116.84 81.28) (end 118.11 80.01) (width 0.25) (layer B.Cu) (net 7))
 (segment (start 125.73 80.01) (end 127 78.74) (width 0.25) (layer B.Cu) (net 7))
 (segment (start 118.11 80.01) (end 125.73 80.01) (width 0.25) (layer B.Cu) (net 7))
 (segment (start 95.25 58.42) (end 96.52 59.69) (width 0.25) (layer B.Cu) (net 7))
 (segment (start 93.345 58.42) (end 95.25 58.42) (width 0.25) (layer B.Cu) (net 7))
 (segment (start 92.71 59.055) (end 93.345 58.42) (width 0.25) (layer B.Cu) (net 7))
 (segment (start 92.71 64.77) (end 92.71 59.055) (width 0.25) (layer B.Cu) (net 7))
 (segment (start 125.095 76.835) (end 111.125 76.835) (width 0.25) (layer B.Cu) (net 7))
 (segment (start 111.125 76.835) (end 110.49 76.2) (width 0.25) (layer B.Cu) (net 7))
 (segment (start 127 78.74) (end 125.095 76.835) (width 0.25) (layer B.Cu) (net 7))
 (segment (start 104.14 76.2) (end 92.71 64.77) (width 0.25) (layer B.Cu) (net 7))
 (segment (start 110.49 76.2) (end 104.14 76.2) (width 0.25) (layer B.Cu) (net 7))
 (segment (start 119.38 81.28) (end 118.11 80.01) (width 0.25) (layer F.Cu) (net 19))
 (segment (start 118.11 78.74) (end 118.11 78.270998) (width 0.25) (layer F.Cu) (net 19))
 (segment (start 118.11 80.01) (end 118.11 78.74) (width 0.25) (layer F.Cu) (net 19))
 (segment (start 118.11 77.47) (end 118.11 78.74) (width 0.25) (layer F.Cu) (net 19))
 (segment (start 117.475 76.835) (end 118.11 77.47) (width 0.25) (layer F.Cu) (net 19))
 (segment (start 104.775 76.835) (end 117.475 76.835) (width 0.25) (layer F.Cu) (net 19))
 (segment (start 93.98 66.04) (end 104.775 76.835) (width 0.25) (layer F.Cu) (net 19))
 (segment (start 93.98 62.23) (end 93.98 66.04) (width 0.25) (layer F.Cu) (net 19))
 (segment (start 120.65 80.01) (end 120.65 77.47) (width 0.25) (layer F.Cu) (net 4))
 (segment (start 121.92 81.28) (end 120.65 80.01) (width 0.25) (layer F.Cu) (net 4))
 (segment (start 104.14 59.69) (end 102.87 60.96) (width 0.25) (layer F.Cu) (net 4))
 (segment (start 102.87 73.66) (end 105.41 76.2) (width 0.25) (layer F.Cu) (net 4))
 (segment (start 102.87 60.96) (end 102.87 73.66) (width 0.25) (layer F.Cu) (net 4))
 (segment (start 105.41 76.2) (end 119.38 76.2) (width 0.25) (layer F.Cu) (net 4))
 (segment (start 119.38 76.2) (end 120.65 77.47) (width 0.25) (layer F.Cu) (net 4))
 (segment (start 124.46 81.28) (end 123.19 80.01) (width 0.25) (layer F.Cu) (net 15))
 (segment (start 123.19 80.01) (end 123.19 77.47) (width 0.25) (layer F.Cu) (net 15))
 (segment (start 123.19 77.47) (end 121.285 75.565) (width 0.25) (layer F.Cu) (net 15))
 (segment (start 121.285 75.565) (end 106.045 75.565) (width 0.25) (layer F.Cu) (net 15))
 (segment (start 104.14 62.23) (end 104.14 73.66) (width 0.25) (layer F.Cu) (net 15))
 (segment (start 106.045 75.565) (end 104.14 73.66) (width 0.25) (layer F.Cu) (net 15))
 (segment (start 127 81.28) (end 125.73 80.01) (width 0.25) (layer F.Cu) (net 5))
 (segment (start 125.73 80.01) (end 125.73 78.105) (width 0.25) (layer F.Cu) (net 5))
 (segment (start 125.73 78.105) (end 118.745 71.12) (width 0.25) (layer F.Cu) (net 5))
 (segment (start 118.745 71.12) (end 118.4275 70.8025) (width 0.25) (layer F.Cu) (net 5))
 (via (at 118.4275 70.8025) (size 0.8) (drill 0.4) (layers F.Cu B.Cu) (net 5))
 (segment (start 102.87 60.96) (end 101.6 59.69) (width 0.25) (layer B.Cu) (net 5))
 (segment (start 118.4275 70.8025) (end 106.3625 70.8025) (width 0.25) (layer B.Cu) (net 5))
 (segment (start 102.87 67.31) (end 102.87 60.96) (width 0.25) (layer B.Cu) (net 5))
 (segment (start 106.3625 70.8025) (end 102.87 67.31) (width 0.25) (layer B.Cu) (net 5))
 (segment (start 129.54 81.28) (end 128.27 80.01) (width 0.25) (layer F.Cu) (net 16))
 (segment (start 128.27 78.74) (end 128.27 77.47) (width 0.25) (layer F.Cu) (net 16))
 (segment (start 128.27 78.74) (end 128.27 78.270998) (width 0.25) (layer F.Cu) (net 16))
 (segment (start 128.27 80.01) (end 128.27 78.74) (width 0.25) (layer F.Cu) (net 16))
 (segment (start 101.6 62.23) (end 101.6 67.31) (width 0.25) (layer B.Cu) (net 16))
 (segment (start 128.27 77.47) (end 122.555 71.755) (width 0.25) (layer F.Cu) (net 16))
 (segment (start 122.555 71.755) (end 122.555 71.755) (width 0.25) (layer F.Cu) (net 16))
 (via (at 122.555 71.755) (size 0.8) (drill 0.4) (layers F.Cu B.Cu) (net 16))
 (segment (start 106.045 71.755) (end 101.6 67.31) (width 0.25) (layer B.Cu) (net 16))
 (segment (start 122.555 71.755) (end 106.045 71.755) (width 0.25) (layer B.Cu) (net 16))
 (segment (start 132.08 81.28) (end 130.81 80.01) (width 0.25) (layer F.Cu) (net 6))
 (segment (start 130.81 80.01) (end 130.81 77.47) (width 0.25) (layer F.Cu) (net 6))
 (segment (start 130.81 77.47) (end 125.984 72.644) (width 0.25) (layer F.Cu) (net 6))
 (segment (start 125.984 72.644) (end 125.984 72.644) (width 0.25) (layer F.Cu) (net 6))
 (via (at 125.984 72.644) (size 0.8) (drill 0.4) (layers F.Cu B.Cu) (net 6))
 (segment (start 100.33 60.96) (end 99.06 59.69) (width 0.25) (layer B.Cu) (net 6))
 (segment (start 100.33 67.31) (end 100.33 60.96) (width 0.25) (layer B.Cu) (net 6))
 (segment (start 125.984 72.644) (end 105.664 72.644) (width 0.25) (layer B.Cu) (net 6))
 (segment (start 105.664 72.644) (end 100.33 67.31) (width 0.25) (layer B.Cu) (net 6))
 (segment (start 134.62 81.28) (end 133.35 80.01) (width 0.25) (layer F.Cu) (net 17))
 (segment (start 133.35 80.01) (end 133.35 77.47) (width 0.25) (layer F.Cu) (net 17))
 (segment (start 129.54 73.66) (end 129.54 73.66) (width 0.25) (layer F.Cu) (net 17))
 (segment (start 99.06 67.31) (end 99.06 62.23) (width 0.25) (layer B.Cu) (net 17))
 (segment (start 105.41 73.66) (end 99.06 67.31) (width 0.25) (layer B.Cu) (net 17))
 (segment (start 133.35 77.47) (end 129.54 73.66) (width 0.25) (layer F.Cu) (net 17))
 (segment (start 129.54 73.66) (end 129.54 73.66) (width 0.25) (layer F.Cu) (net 17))
 (via (at 129.54 73.66) (size 0.8) (drill 0.4) (layers F.Cu B.Cu) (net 17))
 (segment (start 129.54 73.66) (end 105.41 73.66) (width 0.25) (layer B.Cu) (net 17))
 (segment (start 137.16 81.28) (end 135.89 80.01) (width 0.25) (layer F.Cu) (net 18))
 (segment (start 135.89 80.01) (end 135.89 77.47) (width 0.25) (layer F.Cu) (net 18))
 (segment (start 96.52 66.04) (end 96.52 62.23) (width 0.25) (layer B.Cu) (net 18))
 (segment (start 104.775 74.295) (end 96.52 66.04) (width 0.25) (layer B.Cu) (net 18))
 (segment (start 133.096 74.676) (end 105.156 74.676) (width 0.25) (layer B.Cu) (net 18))
 (segment (start 105.156 74.676) (end 104.648 74.168) (width 0.25) (layer B.Cu) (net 18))
 (segment (start 133.35 74.93) (end 133.096 74.676) (width 0.25) (layer F.Cu) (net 18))
 (via (at 133.096 74.676) (size 0.8) (drill 0.4) (layers F.Cu B.Cu) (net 18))
 (segment (start 135.89 77.47) (end 133.096 74.676) (width 0.25) (layer F.Cu) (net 18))
 (segment (start 139.7 81.28) (end 138.43 80.01) (width 0.25) (layer F.Cu) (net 8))
 (segment (start 138.43 80.01) (end 138.43 77.47) (width 0.25) (layer F.Cu) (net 8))
 (segment (start 138.43 77.47) (end 136.525 75.565) (width 0.25) (layer F.Cu) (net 8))
 (segment (start 136.525 75.565) (end 136.525 75.565) (width 0.25) (layer F.Cu) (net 8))
 (via (at 136.525 75.565) (size 0.8) (drill 0.4) (layers F.Cu B.Cu) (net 8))
 (segment (start 136.525 75.565) (end 104.775 75.565) (width 0.25) (layer B.Cu) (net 8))
 (segment (start 104.775 75.565) (end 95.25 66.04) (width 0.25) (layer B.Cu) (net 8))
 (segment (start 95.25 60.96) (end 93.98 59.69) (width 0.25) (layer B.Cu) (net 8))
 (segment (start 95.25 66.04) (end 95.25 60.96) (width 0.25) (layer B.Cu) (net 8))
 (segment (start 111.76 62.23) (end 114.3 62.23) (width 0.5) (layer B.Cu) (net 3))
 (segment (start 111.76 59.69) (end 111.76 62.23) (width 0.5) (layer B.Cu) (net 3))
 (segment (start 111.76 59.69) (end 114.3 59.69) (width 0.5) (layer B.Cu) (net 3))
 (segment (start 114.3 62.23) (end 114.3 59.69) (width 0.5) (layer B.Cu) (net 3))
 (segment (start 114.3 62.23) (end 117.475 65.405) (width 0.5) (layer F.Cu) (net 3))
 (segment (start 111.76 62.23) (end 116.205 66.675) (width 0.5) (layer F.Cu) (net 3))
 (segment (start 116.205 66.675) (end 123.19 66.675) (width 0.5) (layer F.Cu) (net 3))
 (segment (start 128.365 63.595) (end 124.365 63.595) (width 0.5) (layer F.Cu) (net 3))
 (segment (start 128.365 63.595) (end 131 60.96) (width 0.5) (layer F.Cu) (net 3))
 (segment (start 129.615 64.845) (end 133.5 60.96) (width 0.5) (layer F.Cu) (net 3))
 (segment (start 125.02 64.845) (end 129.615 64.845) (width 0.5) (layer F.Cu) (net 3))
 (segment (start 123.19 66.675) (end 125.02 64.845) (width 0.5) (layer F.Cu) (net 3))
 (segment (start 124.365 63.595) (end 122.555 65.405) (width 0.5) (layer F.Cu) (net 3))
 (segment (start 122.555 65.405) (end 117.475 65.405) (width 0.5) (layer F.Cu) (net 3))
 (segment (start 140.716 82.804) (end 110.744 82.804) (width 0.5) (layer F.Cu) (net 1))
 (segment (start 110.744 82.804) (end 109.22 81.28) (width 0.5) (layer F.Cu) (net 1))
 (segment (start 141.224 82.296) (end 140.716 82.804) (width 0.5) (layer F.Cu) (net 1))
 (segment (start 137.795 72.898) (end 141.224 76.327) (width 0.5) (layer F.Cu) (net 1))
 (segment (start 141.224 76.327) (end 141.224 82.296) (width 0.5) (layer F.Cu) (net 1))
 (segment (start 127 69.85) (end 127.635 69.85) (width 0.5) (layer B.Cu) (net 1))
 (segment (start 137.795 72.898) (end 137.795 69.85) (width 0.5) (layer F.Cu) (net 1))
 (segment (start 127.23 62.23) (end 128.5 60.96) (width 0.5) (layer B.Cu) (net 1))
 (segment (start 106.68 59.69) (end 106.68 62.23) (width 0.5) (layer B.Cu) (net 1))
 (segment (start 119.38 62.23) (end 121.285 62.23) (width 0.5) (layer B.Cu) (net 1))
 (segment (start 119.38 59.69) (end 119.38 62.23) (width 0.5) (layer B.Cu) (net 1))
 (segment (start 119.38 62.23) (end 127.23 62.23) (width 0.5) (layer B.Cu) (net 1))
 (segment (start 108.585 64.135) (end 106.68 62.23) (width 0.5) (layer B.Cu) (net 1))
 (segment (start 119.38 62.23) (end 127 69.85) (width 0.5) (layer B.Cu) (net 1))
 (segment (start 119.38 62.23) (end 117.475 64.135) (width 0.5) (layer B.Cu) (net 1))
 (segment (start 117.475 64.135) (end 108.585 64.135) (width 0.5) (layer B.Cu) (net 1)))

